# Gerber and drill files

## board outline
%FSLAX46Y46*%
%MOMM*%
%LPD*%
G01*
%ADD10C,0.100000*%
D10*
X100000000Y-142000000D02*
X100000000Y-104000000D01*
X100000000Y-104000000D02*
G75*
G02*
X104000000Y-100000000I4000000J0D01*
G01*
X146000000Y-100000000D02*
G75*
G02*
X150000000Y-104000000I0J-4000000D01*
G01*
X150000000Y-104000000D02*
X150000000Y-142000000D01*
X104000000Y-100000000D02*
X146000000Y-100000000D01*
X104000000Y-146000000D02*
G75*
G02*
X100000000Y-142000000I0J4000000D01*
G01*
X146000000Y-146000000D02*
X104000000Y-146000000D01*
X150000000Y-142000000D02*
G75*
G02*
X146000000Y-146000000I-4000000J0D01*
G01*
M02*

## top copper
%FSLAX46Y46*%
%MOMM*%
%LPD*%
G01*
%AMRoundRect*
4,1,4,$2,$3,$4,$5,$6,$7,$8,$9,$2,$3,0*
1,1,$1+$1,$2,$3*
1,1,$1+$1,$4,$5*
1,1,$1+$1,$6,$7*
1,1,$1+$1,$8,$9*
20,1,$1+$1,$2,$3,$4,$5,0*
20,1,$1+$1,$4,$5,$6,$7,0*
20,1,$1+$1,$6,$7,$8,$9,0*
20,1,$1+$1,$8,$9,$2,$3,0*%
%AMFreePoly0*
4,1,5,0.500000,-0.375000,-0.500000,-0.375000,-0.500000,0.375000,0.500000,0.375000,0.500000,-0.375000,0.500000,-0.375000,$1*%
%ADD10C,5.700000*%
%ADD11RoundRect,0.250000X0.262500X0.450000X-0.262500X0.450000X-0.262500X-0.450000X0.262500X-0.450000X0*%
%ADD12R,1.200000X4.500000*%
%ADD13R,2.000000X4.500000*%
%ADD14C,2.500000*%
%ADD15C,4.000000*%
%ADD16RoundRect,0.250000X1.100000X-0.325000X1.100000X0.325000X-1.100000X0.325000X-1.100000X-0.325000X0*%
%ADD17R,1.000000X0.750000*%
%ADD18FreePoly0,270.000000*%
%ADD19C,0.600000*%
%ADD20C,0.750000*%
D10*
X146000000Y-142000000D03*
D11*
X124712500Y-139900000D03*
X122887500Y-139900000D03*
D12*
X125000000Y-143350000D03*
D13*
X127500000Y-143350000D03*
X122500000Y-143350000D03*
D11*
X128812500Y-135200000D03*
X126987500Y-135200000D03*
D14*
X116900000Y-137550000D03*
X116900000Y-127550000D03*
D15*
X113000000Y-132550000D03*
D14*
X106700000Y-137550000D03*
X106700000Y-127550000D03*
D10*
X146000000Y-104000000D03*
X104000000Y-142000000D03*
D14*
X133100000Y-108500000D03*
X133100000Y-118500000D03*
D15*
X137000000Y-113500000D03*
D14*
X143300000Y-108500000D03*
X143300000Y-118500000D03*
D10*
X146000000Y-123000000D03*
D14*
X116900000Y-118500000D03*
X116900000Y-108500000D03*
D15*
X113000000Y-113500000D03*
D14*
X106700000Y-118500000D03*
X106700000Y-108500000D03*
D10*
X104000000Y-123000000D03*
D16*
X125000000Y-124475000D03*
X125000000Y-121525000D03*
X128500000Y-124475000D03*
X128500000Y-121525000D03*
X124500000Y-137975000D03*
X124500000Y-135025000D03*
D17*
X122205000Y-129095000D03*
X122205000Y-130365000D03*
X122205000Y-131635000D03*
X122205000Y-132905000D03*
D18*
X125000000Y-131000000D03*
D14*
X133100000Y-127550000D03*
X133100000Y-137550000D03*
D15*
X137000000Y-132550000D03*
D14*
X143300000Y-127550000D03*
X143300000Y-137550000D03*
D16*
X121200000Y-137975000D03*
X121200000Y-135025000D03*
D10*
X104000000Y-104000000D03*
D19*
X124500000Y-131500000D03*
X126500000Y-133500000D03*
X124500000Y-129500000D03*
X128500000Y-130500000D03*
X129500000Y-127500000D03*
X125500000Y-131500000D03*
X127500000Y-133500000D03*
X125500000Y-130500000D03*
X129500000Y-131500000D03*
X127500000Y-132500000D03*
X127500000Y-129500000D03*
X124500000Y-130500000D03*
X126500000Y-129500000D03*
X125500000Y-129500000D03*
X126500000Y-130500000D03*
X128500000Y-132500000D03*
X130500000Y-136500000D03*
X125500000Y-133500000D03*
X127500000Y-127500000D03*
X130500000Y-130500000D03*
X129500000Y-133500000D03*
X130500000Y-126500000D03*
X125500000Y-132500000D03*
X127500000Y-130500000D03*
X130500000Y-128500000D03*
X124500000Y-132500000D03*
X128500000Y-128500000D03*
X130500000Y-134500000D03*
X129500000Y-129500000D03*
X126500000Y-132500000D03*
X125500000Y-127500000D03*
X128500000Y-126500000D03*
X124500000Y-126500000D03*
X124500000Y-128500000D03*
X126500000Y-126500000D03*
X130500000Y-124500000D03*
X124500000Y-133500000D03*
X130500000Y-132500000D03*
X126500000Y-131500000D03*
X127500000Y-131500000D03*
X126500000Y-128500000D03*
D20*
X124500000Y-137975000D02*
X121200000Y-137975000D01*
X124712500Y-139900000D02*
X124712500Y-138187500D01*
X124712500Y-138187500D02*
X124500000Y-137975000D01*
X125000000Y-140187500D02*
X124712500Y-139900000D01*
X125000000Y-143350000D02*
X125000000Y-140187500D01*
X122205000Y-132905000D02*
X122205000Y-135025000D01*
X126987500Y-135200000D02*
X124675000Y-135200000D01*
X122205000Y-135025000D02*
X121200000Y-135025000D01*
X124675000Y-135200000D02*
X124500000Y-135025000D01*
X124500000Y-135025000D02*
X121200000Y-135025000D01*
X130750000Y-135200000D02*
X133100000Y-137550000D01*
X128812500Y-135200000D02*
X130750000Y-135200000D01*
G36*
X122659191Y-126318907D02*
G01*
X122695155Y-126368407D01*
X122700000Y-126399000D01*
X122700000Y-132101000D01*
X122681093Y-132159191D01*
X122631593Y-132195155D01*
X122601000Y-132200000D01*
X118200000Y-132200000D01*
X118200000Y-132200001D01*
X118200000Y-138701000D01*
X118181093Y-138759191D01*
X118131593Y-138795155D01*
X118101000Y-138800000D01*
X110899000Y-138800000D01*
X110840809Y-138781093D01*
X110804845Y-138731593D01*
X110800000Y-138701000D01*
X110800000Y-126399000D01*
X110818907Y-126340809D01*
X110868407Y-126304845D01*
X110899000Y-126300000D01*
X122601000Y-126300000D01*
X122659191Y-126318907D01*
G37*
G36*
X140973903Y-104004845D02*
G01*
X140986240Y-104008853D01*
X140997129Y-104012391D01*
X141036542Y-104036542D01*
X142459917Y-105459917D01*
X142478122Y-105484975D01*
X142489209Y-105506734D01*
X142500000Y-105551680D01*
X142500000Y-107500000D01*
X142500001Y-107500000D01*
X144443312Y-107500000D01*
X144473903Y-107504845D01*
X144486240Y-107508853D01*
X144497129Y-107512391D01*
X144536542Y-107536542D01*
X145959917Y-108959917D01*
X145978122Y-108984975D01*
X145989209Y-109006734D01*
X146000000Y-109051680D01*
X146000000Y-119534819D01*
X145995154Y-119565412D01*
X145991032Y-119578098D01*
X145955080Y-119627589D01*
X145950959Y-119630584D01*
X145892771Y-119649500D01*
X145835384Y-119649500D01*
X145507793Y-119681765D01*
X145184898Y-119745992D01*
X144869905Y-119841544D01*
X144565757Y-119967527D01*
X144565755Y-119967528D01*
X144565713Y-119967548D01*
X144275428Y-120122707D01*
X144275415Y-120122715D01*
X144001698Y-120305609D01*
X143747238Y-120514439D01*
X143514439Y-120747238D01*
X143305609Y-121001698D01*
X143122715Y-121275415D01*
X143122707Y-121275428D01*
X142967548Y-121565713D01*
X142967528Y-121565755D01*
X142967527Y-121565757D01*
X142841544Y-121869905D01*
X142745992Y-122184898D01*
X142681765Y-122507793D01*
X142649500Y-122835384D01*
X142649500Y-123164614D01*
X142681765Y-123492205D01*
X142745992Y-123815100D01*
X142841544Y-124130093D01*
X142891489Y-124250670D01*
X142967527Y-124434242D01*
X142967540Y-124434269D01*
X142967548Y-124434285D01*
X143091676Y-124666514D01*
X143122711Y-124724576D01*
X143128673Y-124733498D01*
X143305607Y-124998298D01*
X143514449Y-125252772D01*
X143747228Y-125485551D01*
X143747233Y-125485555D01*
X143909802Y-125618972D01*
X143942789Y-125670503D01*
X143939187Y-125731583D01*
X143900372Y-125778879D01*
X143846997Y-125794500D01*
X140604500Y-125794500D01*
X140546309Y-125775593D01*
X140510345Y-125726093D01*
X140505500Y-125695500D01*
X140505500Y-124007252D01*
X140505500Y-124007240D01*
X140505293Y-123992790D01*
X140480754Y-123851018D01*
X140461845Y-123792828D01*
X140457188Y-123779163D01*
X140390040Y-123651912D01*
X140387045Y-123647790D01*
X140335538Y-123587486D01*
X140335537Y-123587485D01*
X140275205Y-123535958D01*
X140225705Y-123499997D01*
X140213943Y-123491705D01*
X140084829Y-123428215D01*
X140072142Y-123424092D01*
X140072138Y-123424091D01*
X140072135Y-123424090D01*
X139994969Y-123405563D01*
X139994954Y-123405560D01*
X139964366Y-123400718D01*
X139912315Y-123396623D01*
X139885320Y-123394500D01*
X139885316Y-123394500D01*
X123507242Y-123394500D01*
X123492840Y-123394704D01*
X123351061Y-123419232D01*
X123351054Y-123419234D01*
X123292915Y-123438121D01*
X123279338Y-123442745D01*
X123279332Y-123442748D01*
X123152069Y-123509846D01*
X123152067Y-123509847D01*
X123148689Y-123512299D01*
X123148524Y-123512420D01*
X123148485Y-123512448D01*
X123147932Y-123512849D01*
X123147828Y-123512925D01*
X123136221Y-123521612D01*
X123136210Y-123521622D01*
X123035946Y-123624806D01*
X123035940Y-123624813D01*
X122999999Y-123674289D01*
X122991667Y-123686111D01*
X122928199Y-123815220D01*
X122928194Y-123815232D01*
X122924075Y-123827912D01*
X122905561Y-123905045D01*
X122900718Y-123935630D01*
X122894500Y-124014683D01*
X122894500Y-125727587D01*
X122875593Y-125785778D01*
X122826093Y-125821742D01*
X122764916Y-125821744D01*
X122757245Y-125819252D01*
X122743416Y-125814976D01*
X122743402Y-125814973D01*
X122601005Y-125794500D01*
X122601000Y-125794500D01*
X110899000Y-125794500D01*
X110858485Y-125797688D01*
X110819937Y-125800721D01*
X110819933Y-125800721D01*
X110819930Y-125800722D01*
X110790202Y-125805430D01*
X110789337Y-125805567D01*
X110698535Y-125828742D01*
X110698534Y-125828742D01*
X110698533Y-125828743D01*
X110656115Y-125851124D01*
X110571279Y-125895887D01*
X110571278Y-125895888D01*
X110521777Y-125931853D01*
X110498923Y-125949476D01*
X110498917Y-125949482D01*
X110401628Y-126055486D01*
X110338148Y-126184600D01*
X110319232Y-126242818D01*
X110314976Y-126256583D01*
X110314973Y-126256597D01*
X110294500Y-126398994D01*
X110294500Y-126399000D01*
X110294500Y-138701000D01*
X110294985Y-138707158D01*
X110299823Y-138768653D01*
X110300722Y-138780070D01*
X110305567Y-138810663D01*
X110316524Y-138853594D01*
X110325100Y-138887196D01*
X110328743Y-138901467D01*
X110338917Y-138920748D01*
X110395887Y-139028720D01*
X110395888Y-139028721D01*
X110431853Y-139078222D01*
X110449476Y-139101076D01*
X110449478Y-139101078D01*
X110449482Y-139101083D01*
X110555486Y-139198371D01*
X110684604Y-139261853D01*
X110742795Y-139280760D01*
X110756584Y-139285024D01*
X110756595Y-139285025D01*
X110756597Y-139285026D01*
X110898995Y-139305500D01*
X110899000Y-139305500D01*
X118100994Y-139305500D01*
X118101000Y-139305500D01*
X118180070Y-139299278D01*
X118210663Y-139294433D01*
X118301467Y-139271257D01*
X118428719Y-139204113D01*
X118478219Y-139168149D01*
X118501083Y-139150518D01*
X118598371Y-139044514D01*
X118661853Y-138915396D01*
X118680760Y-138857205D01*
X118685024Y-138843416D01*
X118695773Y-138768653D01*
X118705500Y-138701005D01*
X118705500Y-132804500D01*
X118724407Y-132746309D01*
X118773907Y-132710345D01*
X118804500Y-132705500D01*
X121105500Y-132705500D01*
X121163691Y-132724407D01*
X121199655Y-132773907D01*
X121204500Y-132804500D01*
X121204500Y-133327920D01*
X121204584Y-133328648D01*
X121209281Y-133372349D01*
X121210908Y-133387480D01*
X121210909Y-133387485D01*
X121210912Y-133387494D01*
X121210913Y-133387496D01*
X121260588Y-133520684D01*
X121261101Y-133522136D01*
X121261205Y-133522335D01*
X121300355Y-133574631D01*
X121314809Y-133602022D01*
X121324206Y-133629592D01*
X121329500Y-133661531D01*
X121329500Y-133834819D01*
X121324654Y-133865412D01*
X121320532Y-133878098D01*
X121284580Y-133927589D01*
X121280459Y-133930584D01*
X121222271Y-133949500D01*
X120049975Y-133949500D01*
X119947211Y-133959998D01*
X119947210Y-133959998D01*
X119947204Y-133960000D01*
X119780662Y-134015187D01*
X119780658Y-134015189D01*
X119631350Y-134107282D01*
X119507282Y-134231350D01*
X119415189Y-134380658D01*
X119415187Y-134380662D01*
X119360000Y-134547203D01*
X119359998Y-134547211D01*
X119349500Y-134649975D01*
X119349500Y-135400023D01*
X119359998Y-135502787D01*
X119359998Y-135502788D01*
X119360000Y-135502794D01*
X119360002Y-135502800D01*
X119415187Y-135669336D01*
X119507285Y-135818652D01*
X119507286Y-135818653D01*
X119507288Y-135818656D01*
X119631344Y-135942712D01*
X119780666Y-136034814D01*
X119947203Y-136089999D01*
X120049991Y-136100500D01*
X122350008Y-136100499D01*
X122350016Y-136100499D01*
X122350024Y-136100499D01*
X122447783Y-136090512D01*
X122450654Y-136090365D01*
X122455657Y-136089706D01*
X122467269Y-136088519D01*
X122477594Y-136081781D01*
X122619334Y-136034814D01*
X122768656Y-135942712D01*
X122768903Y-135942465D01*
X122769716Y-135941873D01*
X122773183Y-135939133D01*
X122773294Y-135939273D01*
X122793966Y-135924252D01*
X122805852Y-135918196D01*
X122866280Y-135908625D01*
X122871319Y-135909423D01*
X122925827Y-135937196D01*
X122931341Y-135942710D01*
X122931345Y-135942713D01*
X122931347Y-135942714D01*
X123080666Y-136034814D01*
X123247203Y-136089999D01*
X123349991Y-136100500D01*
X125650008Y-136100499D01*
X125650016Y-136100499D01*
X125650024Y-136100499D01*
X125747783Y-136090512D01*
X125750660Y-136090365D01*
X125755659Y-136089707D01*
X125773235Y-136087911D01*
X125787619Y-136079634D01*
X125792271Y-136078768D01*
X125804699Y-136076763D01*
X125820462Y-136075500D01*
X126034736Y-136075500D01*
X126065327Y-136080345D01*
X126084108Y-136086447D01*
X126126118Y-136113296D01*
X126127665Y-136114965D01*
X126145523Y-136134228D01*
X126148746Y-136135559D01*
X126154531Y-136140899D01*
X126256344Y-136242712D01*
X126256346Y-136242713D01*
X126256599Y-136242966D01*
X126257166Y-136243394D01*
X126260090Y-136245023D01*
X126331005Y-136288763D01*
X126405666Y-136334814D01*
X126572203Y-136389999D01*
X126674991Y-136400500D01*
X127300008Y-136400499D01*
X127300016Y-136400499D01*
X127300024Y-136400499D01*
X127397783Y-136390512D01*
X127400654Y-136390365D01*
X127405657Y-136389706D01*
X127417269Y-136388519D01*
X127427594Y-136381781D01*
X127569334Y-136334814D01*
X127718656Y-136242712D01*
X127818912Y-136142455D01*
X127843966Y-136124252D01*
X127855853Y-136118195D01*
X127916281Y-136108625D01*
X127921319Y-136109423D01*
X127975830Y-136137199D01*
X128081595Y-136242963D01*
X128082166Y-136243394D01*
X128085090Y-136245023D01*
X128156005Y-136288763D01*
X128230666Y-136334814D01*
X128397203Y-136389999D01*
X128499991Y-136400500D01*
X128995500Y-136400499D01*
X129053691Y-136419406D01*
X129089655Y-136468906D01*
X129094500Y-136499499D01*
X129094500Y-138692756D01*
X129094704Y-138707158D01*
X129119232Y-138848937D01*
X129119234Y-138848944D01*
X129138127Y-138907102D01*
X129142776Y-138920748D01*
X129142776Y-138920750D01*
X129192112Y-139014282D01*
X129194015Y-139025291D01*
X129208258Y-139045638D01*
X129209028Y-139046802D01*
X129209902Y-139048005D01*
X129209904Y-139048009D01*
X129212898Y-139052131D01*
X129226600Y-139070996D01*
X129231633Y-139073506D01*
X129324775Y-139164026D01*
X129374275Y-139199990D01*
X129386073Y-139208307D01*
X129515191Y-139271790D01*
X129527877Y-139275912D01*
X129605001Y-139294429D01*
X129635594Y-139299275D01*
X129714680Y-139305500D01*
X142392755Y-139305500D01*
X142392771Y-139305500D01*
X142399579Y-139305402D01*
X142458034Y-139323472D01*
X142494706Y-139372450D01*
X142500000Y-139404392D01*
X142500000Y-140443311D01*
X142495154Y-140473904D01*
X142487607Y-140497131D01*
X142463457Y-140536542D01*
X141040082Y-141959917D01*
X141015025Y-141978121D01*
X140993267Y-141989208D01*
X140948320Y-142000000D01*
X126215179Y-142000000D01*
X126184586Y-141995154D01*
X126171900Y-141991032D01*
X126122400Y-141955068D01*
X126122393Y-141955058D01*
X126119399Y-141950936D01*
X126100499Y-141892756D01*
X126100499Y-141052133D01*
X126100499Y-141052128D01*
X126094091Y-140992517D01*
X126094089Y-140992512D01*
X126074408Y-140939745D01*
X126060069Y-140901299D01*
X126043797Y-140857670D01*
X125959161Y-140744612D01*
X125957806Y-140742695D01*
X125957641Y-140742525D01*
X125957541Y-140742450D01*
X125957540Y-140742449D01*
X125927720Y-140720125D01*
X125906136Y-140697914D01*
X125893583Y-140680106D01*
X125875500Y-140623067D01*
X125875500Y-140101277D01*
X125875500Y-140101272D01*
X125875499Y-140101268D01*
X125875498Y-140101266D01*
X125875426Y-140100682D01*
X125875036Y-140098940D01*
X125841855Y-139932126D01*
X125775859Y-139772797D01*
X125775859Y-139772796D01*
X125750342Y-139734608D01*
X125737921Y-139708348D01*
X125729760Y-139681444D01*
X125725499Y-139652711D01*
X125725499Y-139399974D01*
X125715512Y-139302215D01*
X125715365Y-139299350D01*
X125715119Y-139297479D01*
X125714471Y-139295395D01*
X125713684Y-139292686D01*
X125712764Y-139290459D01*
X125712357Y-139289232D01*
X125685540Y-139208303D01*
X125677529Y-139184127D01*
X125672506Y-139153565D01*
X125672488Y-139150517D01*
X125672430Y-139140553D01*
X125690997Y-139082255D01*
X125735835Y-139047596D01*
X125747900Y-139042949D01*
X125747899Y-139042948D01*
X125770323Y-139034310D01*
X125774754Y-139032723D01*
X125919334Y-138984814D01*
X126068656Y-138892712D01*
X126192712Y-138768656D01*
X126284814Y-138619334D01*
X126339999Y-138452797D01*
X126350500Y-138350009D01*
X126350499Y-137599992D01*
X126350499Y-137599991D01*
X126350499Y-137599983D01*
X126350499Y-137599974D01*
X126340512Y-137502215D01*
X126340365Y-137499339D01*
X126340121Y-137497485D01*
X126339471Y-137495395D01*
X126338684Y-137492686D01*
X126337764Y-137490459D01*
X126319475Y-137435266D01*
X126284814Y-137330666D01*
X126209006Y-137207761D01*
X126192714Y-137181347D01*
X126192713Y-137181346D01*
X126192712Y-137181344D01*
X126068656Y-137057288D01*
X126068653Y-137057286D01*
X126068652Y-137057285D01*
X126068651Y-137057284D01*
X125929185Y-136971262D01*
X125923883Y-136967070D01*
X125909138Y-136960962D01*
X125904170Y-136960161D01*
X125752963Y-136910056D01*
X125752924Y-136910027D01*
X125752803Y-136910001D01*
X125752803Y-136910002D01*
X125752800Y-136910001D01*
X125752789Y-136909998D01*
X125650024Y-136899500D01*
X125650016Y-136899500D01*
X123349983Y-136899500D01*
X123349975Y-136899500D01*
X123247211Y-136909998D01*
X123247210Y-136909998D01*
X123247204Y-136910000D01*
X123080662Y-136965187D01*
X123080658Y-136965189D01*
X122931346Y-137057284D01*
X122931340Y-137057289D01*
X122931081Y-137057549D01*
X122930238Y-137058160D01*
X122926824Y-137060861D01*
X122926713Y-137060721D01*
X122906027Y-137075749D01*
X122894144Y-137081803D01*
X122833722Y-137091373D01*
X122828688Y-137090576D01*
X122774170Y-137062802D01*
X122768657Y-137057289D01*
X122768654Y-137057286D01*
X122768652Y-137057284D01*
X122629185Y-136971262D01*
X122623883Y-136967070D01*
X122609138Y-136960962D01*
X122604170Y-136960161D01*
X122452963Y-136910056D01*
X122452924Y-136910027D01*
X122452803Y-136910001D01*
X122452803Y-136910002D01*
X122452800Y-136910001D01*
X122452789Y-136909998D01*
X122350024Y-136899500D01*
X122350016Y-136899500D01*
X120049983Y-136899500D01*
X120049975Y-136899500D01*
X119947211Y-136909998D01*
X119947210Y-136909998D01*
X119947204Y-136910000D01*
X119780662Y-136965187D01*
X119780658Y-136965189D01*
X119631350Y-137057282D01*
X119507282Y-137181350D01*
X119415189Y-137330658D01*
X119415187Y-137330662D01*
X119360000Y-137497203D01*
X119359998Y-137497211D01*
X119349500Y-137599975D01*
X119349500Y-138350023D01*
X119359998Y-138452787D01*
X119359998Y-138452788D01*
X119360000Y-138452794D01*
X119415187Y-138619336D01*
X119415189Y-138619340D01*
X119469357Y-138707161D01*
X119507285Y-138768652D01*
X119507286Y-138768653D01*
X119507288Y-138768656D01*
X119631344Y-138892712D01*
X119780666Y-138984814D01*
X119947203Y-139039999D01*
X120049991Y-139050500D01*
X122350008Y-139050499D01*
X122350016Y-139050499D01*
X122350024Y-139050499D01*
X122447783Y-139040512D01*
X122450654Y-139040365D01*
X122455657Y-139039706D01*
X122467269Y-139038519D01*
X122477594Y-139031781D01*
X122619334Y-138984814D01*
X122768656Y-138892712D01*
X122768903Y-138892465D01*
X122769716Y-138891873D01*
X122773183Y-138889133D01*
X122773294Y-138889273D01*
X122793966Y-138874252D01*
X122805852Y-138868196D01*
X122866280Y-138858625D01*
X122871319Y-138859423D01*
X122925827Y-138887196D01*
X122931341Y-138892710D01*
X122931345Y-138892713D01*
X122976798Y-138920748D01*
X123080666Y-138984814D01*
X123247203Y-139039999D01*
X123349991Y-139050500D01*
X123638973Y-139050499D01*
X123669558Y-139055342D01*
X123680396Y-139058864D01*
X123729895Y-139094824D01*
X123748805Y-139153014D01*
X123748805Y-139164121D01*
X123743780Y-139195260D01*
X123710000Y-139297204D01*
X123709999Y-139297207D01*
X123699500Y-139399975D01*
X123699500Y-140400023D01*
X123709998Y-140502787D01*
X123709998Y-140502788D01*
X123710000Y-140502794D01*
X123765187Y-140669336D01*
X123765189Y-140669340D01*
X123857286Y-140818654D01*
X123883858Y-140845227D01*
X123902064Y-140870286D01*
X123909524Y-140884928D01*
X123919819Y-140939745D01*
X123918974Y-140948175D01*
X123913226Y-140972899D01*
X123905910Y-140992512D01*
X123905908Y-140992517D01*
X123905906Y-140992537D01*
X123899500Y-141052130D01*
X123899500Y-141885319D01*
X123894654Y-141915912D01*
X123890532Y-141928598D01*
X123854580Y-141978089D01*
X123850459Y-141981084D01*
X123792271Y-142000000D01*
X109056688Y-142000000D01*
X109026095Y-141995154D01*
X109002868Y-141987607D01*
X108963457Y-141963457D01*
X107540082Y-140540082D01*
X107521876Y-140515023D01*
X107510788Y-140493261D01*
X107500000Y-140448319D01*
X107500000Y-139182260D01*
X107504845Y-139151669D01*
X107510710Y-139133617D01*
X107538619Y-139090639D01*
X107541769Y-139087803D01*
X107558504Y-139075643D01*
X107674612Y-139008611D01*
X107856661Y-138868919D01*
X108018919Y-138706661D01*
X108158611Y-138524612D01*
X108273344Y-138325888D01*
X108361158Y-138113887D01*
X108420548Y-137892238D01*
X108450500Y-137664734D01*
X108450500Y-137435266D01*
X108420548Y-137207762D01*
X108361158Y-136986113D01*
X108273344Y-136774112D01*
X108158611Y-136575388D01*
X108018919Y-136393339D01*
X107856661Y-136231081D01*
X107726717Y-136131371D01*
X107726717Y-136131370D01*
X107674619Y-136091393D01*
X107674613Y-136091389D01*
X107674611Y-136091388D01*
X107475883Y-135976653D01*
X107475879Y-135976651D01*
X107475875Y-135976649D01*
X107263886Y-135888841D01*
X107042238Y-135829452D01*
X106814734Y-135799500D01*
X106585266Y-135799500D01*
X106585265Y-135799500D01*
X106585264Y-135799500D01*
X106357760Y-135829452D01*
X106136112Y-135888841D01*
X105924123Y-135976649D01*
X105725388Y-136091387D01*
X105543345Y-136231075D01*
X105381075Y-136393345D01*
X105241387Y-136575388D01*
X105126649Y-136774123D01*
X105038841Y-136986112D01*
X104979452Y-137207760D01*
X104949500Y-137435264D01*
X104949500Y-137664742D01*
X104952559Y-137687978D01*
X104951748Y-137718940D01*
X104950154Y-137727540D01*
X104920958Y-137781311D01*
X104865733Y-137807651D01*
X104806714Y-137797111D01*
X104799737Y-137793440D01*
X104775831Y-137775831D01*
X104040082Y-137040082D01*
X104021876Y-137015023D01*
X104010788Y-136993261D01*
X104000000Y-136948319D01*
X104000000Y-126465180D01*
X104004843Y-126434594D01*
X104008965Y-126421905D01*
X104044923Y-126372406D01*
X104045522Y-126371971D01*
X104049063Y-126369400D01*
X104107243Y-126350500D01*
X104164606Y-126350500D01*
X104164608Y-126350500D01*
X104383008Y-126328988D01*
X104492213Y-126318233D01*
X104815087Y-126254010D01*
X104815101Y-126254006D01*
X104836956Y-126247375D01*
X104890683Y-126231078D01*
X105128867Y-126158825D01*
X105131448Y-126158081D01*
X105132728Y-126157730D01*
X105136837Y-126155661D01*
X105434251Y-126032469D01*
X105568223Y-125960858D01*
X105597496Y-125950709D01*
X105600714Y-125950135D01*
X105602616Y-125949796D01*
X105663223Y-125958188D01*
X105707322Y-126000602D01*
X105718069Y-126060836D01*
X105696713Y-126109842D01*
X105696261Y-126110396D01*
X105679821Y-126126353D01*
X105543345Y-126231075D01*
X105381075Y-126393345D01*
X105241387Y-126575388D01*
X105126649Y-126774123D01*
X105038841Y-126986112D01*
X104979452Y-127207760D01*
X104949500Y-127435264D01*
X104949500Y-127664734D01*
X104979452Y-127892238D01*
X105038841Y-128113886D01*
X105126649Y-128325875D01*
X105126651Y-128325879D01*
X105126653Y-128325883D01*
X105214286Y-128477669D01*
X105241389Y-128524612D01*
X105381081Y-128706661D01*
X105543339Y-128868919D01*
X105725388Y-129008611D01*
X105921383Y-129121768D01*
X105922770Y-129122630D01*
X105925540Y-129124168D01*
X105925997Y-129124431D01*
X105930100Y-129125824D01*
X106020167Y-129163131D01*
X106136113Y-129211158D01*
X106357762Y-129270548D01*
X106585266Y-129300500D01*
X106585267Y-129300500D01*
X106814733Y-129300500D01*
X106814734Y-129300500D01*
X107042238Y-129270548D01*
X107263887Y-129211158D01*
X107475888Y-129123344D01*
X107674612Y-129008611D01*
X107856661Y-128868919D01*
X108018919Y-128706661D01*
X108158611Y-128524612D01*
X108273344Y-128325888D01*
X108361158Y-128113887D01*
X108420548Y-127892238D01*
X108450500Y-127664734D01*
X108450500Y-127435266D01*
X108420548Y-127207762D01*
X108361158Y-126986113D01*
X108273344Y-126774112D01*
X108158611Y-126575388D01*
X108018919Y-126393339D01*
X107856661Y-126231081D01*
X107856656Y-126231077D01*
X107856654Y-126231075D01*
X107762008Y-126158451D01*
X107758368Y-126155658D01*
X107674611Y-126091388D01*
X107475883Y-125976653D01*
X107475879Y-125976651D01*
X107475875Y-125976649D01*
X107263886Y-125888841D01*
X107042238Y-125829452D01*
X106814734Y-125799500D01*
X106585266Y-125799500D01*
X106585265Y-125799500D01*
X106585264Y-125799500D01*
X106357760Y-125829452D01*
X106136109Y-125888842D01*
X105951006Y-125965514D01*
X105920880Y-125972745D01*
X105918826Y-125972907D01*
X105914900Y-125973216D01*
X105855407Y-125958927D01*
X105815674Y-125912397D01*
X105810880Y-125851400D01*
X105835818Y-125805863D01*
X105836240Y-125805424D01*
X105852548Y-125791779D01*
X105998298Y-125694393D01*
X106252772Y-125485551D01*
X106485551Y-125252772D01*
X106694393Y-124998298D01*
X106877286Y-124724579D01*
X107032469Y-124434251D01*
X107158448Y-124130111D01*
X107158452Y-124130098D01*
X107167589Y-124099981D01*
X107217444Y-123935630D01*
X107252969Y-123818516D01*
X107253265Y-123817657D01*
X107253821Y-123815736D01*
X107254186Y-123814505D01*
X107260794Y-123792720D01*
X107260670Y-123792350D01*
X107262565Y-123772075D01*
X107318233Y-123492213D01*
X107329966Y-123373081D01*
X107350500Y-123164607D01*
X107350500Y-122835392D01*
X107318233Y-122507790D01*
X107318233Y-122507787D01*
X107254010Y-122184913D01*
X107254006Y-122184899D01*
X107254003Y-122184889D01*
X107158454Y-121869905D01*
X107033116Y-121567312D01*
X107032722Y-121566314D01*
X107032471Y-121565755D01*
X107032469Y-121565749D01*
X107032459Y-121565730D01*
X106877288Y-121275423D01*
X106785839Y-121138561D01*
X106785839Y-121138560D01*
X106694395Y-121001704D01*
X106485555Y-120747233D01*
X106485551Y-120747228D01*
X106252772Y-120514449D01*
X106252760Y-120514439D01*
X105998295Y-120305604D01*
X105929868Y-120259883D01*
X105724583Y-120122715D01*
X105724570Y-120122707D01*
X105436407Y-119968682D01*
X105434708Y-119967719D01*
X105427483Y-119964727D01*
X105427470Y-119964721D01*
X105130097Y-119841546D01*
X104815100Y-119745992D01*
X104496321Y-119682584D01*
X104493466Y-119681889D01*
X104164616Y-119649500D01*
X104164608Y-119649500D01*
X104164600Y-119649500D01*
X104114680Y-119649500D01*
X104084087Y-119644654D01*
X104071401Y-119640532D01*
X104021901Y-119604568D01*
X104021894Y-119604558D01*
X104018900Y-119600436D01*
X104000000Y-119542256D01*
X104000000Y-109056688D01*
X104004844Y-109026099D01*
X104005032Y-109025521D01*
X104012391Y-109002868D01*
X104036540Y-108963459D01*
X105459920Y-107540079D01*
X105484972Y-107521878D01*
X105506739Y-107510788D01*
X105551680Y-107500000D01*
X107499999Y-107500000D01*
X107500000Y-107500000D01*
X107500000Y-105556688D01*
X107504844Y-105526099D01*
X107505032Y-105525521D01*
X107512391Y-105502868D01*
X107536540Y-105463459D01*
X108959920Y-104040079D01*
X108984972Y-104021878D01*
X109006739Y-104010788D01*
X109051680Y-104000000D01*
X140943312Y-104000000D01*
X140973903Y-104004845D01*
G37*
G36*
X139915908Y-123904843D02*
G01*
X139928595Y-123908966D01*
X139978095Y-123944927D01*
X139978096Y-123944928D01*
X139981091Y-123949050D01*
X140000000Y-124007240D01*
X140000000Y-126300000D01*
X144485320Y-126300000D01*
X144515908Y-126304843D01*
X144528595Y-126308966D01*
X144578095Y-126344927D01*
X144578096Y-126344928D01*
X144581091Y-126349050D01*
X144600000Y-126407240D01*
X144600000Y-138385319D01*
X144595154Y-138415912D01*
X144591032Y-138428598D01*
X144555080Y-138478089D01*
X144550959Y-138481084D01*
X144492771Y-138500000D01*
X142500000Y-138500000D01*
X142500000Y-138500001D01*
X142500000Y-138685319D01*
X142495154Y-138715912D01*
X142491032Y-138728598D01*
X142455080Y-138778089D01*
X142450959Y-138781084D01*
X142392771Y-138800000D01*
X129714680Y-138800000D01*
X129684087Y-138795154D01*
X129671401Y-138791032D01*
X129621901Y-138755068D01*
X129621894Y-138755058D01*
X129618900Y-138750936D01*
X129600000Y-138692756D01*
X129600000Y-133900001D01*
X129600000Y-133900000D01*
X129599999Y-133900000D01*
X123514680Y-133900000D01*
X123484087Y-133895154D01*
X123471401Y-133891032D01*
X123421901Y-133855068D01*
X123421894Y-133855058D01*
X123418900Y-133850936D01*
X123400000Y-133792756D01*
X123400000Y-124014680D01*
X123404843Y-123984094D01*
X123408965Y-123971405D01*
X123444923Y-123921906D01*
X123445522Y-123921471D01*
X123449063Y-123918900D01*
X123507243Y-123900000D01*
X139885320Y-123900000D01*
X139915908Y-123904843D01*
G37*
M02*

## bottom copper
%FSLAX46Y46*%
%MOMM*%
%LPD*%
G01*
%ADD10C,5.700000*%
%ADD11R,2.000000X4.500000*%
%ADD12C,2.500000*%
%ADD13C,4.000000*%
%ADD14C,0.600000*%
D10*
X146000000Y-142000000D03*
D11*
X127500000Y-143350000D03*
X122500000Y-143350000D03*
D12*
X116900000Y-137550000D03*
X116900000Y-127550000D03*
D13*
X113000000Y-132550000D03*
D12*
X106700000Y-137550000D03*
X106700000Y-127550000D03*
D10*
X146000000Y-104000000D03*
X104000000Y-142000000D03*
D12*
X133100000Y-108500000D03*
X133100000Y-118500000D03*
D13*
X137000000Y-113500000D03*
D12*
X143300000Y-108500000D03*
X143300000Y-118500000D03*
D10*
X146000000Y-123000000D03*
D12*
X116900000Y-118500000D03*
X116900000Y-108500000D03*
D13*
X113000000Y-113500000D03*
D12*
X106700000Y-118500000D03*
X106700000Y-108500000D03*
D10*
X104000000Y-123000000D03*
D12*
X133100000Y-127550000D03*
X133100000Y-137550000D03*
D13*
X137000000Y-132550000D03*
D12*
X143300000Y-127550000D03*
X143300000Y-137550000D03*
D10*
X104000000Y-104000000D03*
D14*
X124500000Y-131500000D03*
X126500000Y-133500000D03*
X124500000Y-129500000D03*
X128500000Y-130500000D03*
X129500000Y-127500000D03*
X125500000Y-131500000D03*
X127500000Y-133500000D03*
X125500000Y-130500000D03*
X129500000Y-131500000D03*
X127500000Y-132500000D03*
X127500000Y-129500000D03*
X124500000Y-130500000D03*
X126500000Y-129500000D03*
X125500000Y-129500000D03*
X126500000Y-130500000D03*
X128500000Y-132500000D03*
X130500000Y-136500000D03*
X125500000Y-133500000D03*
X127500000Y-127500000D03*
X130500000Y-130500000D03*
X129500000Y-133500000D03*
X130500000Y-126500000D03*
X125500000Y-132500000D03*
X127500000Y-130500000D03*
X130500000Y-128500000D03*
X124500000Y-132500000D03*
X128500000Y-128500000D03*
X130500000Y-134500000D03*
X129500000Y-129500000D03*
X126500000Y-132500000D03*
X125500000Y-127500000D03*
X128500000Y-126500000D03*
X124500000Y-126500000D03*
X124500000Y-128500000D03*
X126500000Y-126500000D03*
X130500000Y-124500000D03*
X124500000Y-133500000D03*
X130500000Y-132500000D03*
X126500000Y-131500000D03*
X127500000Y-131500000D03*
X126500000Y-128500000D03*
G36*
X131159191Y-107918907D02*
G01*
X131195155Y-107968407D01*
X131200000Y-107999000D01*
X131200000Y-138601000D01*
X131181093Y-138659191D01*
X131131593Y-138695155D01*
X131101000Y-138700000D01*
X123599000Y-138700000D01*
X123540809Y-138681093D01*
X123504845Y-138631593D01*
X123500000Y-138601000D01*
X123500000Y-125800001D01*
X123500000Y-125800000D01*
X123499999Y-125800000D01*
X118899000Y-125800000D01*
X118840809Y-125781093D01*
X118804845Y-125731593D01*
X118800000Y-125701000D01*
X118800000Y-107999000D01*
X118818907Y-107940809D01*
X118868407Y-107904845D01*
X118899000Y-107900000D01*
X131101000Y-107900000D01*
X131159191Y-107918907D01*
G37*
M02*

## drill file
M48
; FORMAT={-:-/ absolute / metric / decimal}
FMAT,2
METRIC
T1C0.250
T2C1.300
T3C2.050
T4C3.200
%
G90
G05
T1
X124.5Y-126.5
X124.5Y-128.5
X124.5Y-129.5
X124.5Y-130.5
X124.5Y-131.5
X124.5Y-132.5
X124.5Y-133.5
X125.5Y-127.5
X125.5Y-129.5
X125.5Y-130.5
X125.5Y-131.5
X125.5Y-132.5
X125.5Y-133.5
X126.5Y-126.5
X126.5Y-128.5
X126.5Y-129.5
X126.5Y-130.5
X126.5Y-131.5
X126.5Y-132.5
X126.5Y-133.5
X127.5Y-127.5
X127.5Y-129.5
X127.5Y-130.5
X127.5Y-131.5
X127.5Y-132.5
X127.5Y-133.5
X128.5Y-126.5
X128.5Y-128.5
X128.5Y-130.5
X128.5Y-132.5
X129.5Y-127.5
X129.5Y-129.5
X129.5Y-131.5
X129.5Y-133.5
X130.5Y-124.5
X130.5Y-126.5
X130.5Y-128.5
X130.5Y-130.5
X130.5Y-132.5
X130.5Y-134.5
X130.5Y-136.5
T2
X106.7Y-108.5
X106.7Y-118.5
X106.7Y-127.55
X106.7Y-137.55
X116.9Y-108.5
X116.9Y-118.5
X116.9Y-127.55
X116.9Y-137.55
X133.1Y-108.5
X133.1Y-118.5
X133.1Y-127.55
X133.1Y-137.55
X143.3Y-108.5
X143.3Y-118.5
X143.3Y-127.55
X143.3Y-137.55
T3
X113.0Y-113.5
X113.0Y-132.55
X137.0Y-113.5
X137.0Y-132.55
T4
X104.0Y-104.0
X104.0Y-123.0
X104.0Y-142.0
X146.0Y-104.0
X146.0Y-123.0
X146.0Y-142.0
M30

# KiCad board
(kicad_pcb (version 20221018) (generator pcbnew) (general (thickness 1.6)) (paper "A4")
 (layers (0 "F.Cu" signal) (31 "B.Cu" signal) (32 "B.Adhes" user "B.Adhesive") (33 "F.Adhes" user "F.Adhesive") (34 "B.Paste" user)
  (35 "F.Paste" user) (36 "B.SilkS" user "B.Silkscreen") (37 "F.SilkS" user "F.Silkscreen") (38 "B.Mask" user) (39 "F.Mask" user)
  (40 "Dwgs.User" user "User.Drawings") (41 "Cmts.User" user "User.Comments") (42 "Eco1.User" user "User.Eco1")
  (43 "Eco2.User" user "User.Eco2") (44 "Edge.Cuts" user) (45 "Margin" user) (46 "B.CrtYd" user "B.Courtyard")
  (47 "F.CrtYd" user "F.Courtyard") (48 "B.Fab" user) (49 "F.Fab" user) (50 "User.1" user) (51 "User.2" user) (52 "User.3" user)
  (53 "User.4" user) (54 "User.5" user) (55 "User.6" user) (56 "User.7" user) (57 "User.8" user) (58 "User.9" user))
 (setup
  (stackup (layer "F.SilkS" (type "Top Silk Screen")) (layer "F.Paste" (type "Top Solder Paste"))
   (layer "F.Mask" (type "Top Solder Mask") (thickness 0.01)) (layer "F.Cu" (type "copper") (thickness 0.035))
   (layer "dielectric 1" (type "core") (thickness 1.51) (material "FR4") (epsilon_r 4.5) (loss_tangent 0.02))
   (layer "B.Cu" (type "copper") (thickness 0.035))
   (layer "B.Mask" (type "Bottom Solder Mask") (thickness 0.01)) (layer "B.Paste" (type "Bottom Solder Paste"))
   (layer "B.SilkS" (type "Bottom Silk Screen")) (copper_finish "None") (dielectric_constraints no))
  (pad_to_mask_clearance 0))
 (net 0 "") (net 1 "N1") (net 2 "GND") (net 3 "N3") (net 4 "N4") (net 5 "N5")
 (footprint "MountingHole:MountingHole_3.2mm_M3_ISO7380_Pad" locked (layer "F.Cu") (at 146 142)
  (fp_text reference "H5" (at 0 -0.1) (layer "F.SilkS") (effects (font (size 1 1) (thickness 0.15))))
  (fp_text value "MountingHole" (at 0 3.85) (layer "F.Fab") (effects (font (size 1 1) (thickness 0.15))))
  (pad "1" thru_hole circle locked (at 0 0) (size 5.7 5.7) (drill 3.2) (layers "*.Cu" "*.Mask")))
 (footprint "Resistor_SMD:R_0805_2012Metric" (layer "F.Cu") (at 123.8 139.9 180)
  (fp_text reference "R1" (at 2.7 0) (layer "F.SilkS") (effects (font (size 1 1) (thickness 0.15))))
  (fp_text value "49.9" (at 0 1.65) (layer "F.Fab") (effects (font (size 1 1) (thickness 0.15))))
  (pad "1" smd roundrect (at -0.9125 0 180) (size 1.025 1.4) (layers "F.Cu" "F.Paste" "F.Mask") (roundrect_rratio 0.243902439) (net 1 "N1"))
  (pad "2" smd roundrect (at 0.9125 0 180) (size 1.025 1.4) (layers "F.Cu" "F.Paste" "F.Mask") (roundrect_rratio 0.243902439) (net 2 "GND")))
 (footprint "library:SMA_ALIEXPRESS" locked (layer "F.Cu") (at 125 145.6 180)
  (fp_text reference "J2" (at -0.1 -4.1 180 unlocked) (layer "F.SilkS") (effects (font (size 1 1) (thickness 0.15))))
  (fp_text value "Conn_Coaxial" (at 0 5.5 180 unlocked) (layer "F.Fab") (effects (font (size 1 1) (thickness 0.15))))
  (pad "1" smd rect locked (at 0 2.25 180) (size 1.2 4.5) (layers "F.Cu" "F.Paste" "F.Mask") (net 1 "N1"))
  (pad "2" smd rect locked (at -2.5 2.25 180) (size 2 4.5) (layers "F.Cu" "F.Paste" "F.Mask") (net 2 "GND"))
  (pad "2" smd rect locked (at -2.5 2.25 180) (size 2 4.5) (layers "B.Cu" "B.Paste" "B.Mask") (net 2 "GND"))
  (pad "2" smd rect locked (at 2.5 2.25 180) (size 2 4.5) (layers "F.Cu" "F.Paste" "F.Mask") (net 2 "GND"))
  (pad "2" smd rect locked (at 2.5 2.25 180) (size 2 4.5) (layers "B.Cu" "B.Paste" "B.Mask") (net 2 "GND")))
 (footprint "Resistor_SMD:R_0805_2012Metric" (layer "F.Cu") (at 127.9 135.2 180)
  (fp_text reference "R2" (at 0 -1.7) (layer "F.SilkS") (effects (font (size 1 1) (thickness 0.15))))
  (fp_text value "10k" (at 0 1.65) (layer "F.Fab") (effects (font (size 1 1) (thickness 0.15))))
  (pad "1" smd roundrect (at -0.9125 0 180) (size 1.025 1.4) (layers "F.Cu" "F.Paste" "F.Mask") (roundrect_rratio 0.243902439) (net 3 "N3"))
  (pad "2" smd roundrect (at 0.9125 0 180) (size 1.025 1.4) (layers "F.Cu" "F.Paste" "F.Mask") (roundrect_rratio 0.243902439) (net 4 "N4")))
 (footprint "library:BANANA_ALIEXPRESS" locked (layer "F.Cu") (at 113 132.55 180)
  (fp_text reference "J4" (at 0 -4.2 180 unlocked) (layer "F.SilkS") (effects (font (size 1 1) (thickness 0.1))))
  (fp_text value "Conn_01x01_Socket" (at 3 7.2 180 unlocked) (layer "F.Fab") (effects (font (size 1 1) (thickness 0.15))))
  (pad "1" thru_hole circle locked (at -3.9 -5 180) (size 2.5 2.5) (drill 1.3) (layers "*.Cu" "*.Mask") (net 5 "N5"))
  (pad "1" thru_hole circle locked (at -3.9 5 180) (size 2.5 2.5) (drill 1.3) (layers "*.Cu" "*.Mask") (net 5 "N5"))
  (pad "1" thru_hole circle locked (at 0 0 180) (size 4 4) (drill 2.05) (layers "*.Cu" "*.Mask") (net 5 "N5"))
  (pad "1" thru_hole circle locked (at 6.3 -5 180) (size 2.5 2.5) (drill 1.3) (layers "*.Cu" "*.Mask") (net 5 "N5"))
  (pad "1" thru_hole circle locked (at 6.3 5 180) (size 2.5 2.5) (drill 1.3) (layers "*.Cu" "*.Mask") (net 5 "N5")))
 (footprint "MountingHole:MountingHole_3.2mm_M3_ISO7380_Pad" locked (layer "F.Cu") (at 146 104)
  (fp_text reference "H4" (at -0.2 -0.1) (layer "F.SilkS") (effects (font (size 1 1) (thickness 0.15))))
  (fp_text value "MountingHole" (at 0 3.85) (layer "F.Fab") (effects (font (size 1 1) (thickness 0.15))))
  (pad "1" thru_hole circle locked (at 0 0) (size 5.7 5.7) (drill 3.2) (layers "*.Cu" "*.Mask")))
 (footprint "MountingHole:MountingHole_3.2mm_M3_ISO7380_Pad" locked (layer "F.Cu") (at 104 142)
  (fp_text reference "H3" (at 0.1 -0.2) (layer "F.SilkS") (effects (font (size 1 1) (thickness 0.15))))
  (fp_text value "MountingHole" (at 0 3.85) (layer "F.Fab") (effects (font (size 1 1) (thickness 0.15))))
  (pad "1" thru_hole circle locked (at 0 0) (size 5.7 5.7) (drill 3.2) (layers "*.Cu" "*.Mask")))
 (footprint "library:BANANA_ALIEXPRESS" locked (layer "F.Cu") (at 137 113.5)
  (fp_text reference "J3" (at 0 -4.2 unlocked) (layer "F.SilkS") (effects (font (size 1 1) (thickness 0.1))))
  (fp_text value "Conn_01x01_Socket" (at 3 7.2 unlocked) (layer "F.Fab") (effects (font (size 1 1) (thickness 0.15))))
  (pad "1" thru_hole circle locked (at -3.9 -5) (size 2.5 2.5) (drill 1.3) (layers "*.Cu" "*.Mask") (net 2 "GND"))
  (pad "1" thru_hole circle locked (at -3.9 5) (size 2.5 2.5) (drill 1.3) (layers "*.Cu" "*.Mask") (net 2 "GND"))
  (pad "1" thru_hole circle locked (at 0 0) (size 4 4) (drill 2.05) (layers "*.Cu" "*.Mask") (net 2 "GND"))
  (pad "1" thru_hole circle locked (at 6.3 -5) (size 2.5 2.5) (drill 1.3) (layers "*.Cu" "*.Mask") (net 2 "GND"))
  (pad "1" thru_hole circle locked (at 6.3 5) (size 2.5 2.5) (drill 1.3) (layers "*.Cu" "*.Mask") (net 2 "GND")))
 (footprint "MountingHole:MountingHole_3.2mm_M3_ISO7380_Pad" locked (layer "F.Cu") (at 146 123)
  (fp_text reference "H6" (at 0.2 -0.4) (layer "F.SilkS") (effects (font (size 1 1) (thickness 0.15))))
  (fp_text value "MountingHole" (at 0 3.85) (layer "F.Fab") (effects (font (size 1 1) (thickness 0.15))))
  (pad "1" thru_hole circle locked (at 0 0) (size 5.7 5.7) (drill 3.2) (layers "*.Cu" "*.Mask")))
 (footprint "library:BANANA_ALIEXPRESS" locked (layer "F.Cu") (at 113 113.5 180)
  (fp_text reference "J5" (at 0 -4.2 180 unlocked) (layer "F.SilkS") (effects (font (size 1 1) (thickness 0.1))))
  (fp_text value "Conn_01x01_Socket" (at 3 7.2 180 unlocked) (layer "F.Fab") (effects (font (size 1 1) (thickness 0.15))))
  (pad "1" thru_hole circle locked (at -3.9 -5 180) (size 2.5 2.5) (drill 1.3) (layers "*.Cu" "*.Mask") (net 2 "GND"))
  (pad "1" thru_hole circle locked (at -3.9 5 180) (size 2.5 2.5) (drill 1.3) (layers "*.Cu" "*.Mask") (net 2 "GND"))
  (pad "1" thru_hole circle locked (at 0 0 180) (size 4 4) (drill 2.05) (layers "*.Cu" "*.Mask") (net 2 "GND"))
  (pad "1" thru_hole circle locked (at 6.3 -5 180) (size 2.5 2.5) (drill 1.3) (layers "*.Cu" "*.Mask") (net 2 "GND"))
  (pad "1" thru_hole circle locked (at 6.3 5 180) (size 2.5 2.5) (drill 1.3) (layers "*.Cu" "*.Mask") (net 2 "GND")))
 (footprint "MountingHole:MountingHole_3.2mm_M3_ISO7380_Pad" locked (layer "F.Cu") (at 104 123)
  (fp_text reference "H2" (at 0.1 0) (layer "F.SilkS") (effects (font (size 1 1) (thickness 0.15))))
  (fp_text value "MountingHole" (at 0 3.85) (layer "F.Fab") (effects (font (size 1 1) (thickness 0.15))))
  (pad "1" thru_hole circle locked (at 0 0) (size 5.7 5.7) (drill 3.2) (layers "*.Cu" "*.Mask")))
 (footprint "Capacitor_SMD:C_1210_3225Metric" (layer "F.Cu") (at 125 123 90)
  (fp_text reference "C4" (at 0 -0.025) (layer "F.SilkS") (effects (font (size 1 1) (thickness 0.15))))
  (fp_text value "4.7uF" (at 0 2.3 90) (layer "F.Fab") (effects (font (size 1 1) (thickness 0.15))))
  (pad "1" smd roundrect (at -1.475 0 90) (size 1.15 2.7) (layers "F.Cu" "F.Paste" "F.Mask") (roundrect_rratio 0.2173913043) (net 3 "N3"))
  (pad "2" smd roundrect (at 1.475 0 90) (size 1.15 2.7) (layers "F.Cu" "F.Paste" "F.Mask") (roundrect_rratio 0.2173913043) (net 2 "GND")))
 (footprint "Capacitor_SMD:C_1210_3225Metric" (layer "F.Cu") (at 128.5 123 90)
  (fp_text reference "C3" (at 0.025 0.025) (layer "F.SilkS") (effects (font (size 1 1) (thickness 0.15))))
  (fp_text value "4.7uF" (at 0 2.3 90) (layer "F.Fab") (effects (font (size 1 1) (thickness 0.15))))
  (pad "1" smd roundrect (at -1.475 0 90) (size 1.15 2.7) (layers "F.Cu" "F.Paste" "F.Mask") (roundrect_rratio 0.2173913043) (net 3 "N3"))
  (pad "2" smd roundrect (at 1.475 0 90) (size 1.15 2.7) (layers "F.Cu" "F.Paste" "F.Mask") (roundrect_rratio 0.2173913043) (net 2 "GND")))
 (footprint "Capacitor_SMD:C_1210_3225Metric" (layer "F.Cu") (at 124.5 136.5 90)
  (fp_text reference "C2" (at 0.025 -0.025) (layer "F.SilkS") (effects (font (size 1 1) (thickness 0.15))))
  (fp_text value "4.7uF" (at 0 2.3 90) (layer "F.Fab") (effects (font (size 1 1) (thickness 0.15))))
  (pad "1" smd roundrect (at -1.475 0 90) (size 1.15 2.7) (layers "F.Cu" "F.Paste" "F.Mask") (roundrect_rratio 0.2173913043) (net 1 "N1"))
  (pad "2" smd roundrect (at 1.475 0 90) (size 1.15 2.7) (layers "F.Cu" "F.Paste" "F.Mask") (roundrect_rratio 0.2173913043) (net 4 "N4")))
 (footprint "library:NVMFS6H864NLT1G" (layer "F.Cu") (at 125 131)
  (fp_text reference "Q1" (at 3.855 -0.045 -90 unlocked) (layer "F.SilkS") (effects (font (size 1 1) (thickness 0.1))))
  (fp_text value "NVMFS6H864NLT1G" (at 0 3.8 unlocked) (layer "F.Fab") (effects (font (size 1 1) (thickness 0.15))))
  (pad "1" smd rect (at -2.795 -1.905) (size 1 0.75) (layers "F.Cu" "F.Paste" "F.Mask") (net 5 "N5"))
  (pad "2" smd rect (at -2.795 -0.635) (size 1 0.75) (layers "F.Cu" "F.Paste" "F.Mask") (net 5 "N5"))
  (pad "3" smd rect (at -2.795 0.635) (size 1 0.75) (layers "F.Cu" "F.Paste" "F.Mask") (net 5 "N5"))
  (pad "4" smd rect (at -2.795 1.905) (size 1 0.75) (layers "F.Cu" "F.Paste" "F.Mask") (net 4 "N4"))
  (pad "5" smd custom (at 0 0 270) (size 1 0.75) (layers "F.Cu" "F.Paste" "F.Mask") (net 3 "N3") (options (clearance outline) (anchor rect))
   (primitives)))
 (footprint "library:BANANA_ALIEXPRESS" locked (layer "F.Cu") (at 137 132.55)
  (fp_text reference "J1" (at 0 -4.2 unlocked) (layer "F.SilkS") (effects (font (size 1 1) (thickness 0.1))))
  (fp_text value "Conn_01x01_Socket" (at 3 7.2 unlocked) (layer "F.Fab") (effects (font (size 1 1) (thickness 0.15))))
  (pad "1" thru_hole circle locked (at -3.9 -5) (size 2.5 2.5) (drill 1.3) (layers "*.Cu" "*.Mask") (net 3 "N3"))
  (pad "1" thru_hole circle locked (at -3.9 5) (size 2.5 2.5) (drill 1.3) (layers "*.Cu" "*.Mask") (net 3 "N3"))
  (pad "1" thru_hole circle locked (at 0 0) (size 4 4) (drill 2.05) (layers "*.Cu" "*.Mask") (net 3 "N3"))
  (pad "1" thru_hole circle locked (at 6.3 -5) (size 2.5 2.5) (drill 1.3) (layers "*.Cu" "*.Mask") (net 3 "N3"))
  (pad "1" thru_hole circle locked (at 6.3 5) (size 2.5 2.5) (drill 1.3) (layers "*.Cu" "*.Mask") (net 3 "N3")))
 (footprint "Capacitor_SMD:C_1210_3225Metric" (layer "F.Cu") (at 121.2 136.5 90)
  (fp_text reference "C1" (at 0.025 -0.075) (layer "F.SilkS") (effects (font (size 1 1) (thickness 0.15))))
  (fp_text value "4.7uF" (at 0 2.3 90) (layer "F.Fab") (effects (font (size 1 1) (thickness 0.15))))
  (pad "1" smd roundrect (at -1.475 0 90) (size 1.15 2.7) (layers "F.Cu" "F.Paste" "F.Mask") (roundrect_rratio 0.2173913043) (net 1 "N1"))
  (pad "2" smd roundrect (at 1.475 0 90) (size 1.15 2.7) (layers "F.Cu" "F.Paste" "F.Mask") (roundrect_rratio 0.2173913043) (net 4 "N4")))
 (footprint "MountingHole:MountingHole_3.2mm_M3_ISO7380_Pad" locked (layer "F.Cu") (at 104 104)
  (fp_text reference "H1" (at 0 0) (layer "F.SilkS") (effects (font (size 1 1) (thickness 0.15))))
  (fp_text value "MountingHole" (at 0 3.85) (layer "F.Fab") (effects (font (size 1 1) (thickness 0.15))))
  (pad "1" thru_hole circle locked (at 0 0) (size 5.7 5.7) (drill 3.2) (layers "*.Cu" "*.Mask")))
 (gr_line (start 100 142) (end 100 104) (stroke (width 0.1) (type default)) (layer "Edge.Cuts"))
 (gr_arc (start 100 104) (mid 101.171573 101.171573) (end 104 100) (stroke (width 0.1) (type default)) (layer "Edge.Cuts"))
 (gr_arc (start 146 100) (mid 148.828427 101.171573) (end 150 104) (stroke (width 0.1) (type default)) (layer "Edge.Cuts"))
 (gr_line (start 150 104) (end 150 142) (stroke (width 0.1) (type default)) (layer "Edge.Cuts"))
 (gr_line (start 104 100) (end 146 100) (stroke (width 0.1) (type default)) (layer "Edge.Cuts"))
 (gr_arc (start 104 146) (mid 101.171573 144.828427) (end 100 142) (stroke (width 0.1) (type default)) (layer "Edge.Cuts"))
 (gr_line (start 146 146) (end 104 146) (stroke (width 0.1) (type default)) (layer "Edge.Cuts"))
 (gr_arc (start 150 142) (mid 148.828427 144.828427) (end 146 146) (stroke (width 0.1) (type default)) (layer "Edge.Cuts"))
 (segment (start 124.5 137.975) (end 121.2 137.975) (width 0.75) (layer "F.Cu") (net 1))
 (segment (start 124.7125 139.9) (end 124.7125 138.1875) (width 0.75) (layer "F.Cu") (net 1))
 (segment (start 124.7125 138.1875) (end 124.5 137.975) (width 0.75) (layer "F.Cu") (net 1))
 (segment (start 125 140.1875) (end 124.7125 139.9) (width 0.75) (layer "F.Cu") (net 1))
 (segment (start 125 143.35) (end 125 140.1875) (width 0.75) (layer "F.Cu") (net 1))
 (segment (start 122.205 132.905) (end 122.205 135.025) (width 0.75) (layer "F.Cu") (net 4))
 (segment (start 126.9875 135.2) (end 124.675 135.2) (width 0.75) (layer "F.Cu") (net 4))
 (segment (start 122.205 135.025) (end 121.2 135.025) (width 0.75) (layer "F.Cu") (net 4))
 (segment (start 124.675 135.2) (end 124.5 135.025) (width 0.75) (layer "F.Cu") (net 4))
 (segment (start 124.5 135.025) (end 121.2 135.025) (width 0.75) (layer "F.Cu") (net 4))
 (segment (start 130.75 135.2) (end 133.1 137.55) (width 0.75) (layer "F.Cu") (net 3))
 (segment (start 128.8125 135.2) (end 130.75 135.2) (width 0.75) (layer "F.Cu") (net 3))
 (via (at 124.5 131.5) (size 0.6) (drill 0.25) (layers "F.Cu" "B.Cu") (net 3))
 (via (at 126.5 133.5) (size 0.6) (drill 0.25) (layers "F.Cu" "B.Cu") (free) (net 3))
 (via (at 124.5 129.5) (size 0.6) (drill 0.25) (layers "F.Cu" "B.Cu") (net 3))
 (via (at 128.5 130.5) (size 0.6) (drill 0.25) (layers "F.Cu" "B.Cu") (free) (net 3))
 (via (at 129.5 127.5) (size 0.6) (drill 0.25) (layers "F.Cu" "B.Cu") (free) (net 3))
 (via (at 125.5 131.5) (size 0.6) (drill 0.25) (layers "F.Cu" "B.Cu") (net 3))
 (via (at 127.5 133.5) (size 0.6) (drill 0.25) (layers "F.Cu" "B.Cu") (free) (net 3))
 (via (at 125.5 130.5) (size 0.6) (drill 0.25) (layers "F.Cu" "B.Cu") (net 3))
 (via (at 129.5 131.5) (size 0.6) (drill 0.25) (layers "F.Cu" "B.Cu") (free) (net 3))
 (via (at 127.5 132.5) (size 0.6) (drill 0.25) (layers "F.Cu" "B.Cu") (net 3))
 (via (at 127.5 129.5) (size 0.6) (drill 0.25) (layers "F.Cu" "B.Cu") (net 3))
 (via (at 124.5 130.5) (size 0.6) (drill 0.25) (layers "F.Cu" "B.Cu") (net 3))
 (via (at 126.5 129.5) (size 0.6) (drill 0.25) (layers "F.Cu" "B.Cu") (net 3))
 (via (at 125.5 129.5) (size 0.6) (drill 0.25) (layers "F.Cu" "B.Cu") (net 3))
 (via (at 126.5 130.5) (size 0.6) (drill 0.25) (layers "F.Cu" "B.Cu") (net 3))
 (via (at 128.5 132.5) (size 0.6) (drill 0.25) (layers "F.Cu" "B.Cu") (free) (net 3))
 (via (at 130.5 136.5) (size 0.6) (drill 0.25) (layers "F.Cu" "B.Cu") (free) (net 3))
 (via (at 125.5 133.5) (size 0.6) (drill 0.25) (layers "F.Cu" "B.Cu") (free) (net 3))
 (via (at 127.5 127.5) (size 0.6) (drill 0.25) (layers "F.Cu" "B.Cu") (free) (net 3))
 (via (at 130.5 130.5) (size 0.6) (drill 0.25) (layers "F.Cu" "B.Cu") (free) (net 3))
 (via (at 129.5 133.5) (size 0.6) (drill 0.25) (layers "F.Cu" "B.Cu") (free) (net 3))
 (via (at 130.5 126.5) (size 0.6) (drill 0.25) (layers "F.Cu" "B.Cu") (free) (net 3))
 (via (at 125.5 132.5) (size 0.6) (drill 0.25) (layers "F.Cu" "B.Cu") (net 3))
 (via (at 127.5 130.5) (size 0.6) (drill 0.25) (layers "F.Cu" "B.Cu") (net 3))
 (via (at 130.5 128.5) (size 0.6) (drill 0.25) (layers "F.Cu" "B.Cu") (free) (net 3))
 (via (at 124.5 132.5) (size 0.6) (drill 0.25) (layers "F.Cu" "B.Cu") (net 3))
 (via (at 128.5 128.5) (size 0.6) (drill 0.25) (layers "F.Cu" "B.Cu") (free) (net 3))
 (via (at 130.5 134.5) (size 0.6) (drill 0.25) (layers "F.Cu" "B.Cu") (free) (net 3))
 (via (at 129.5 129.5) (size 0.6) (drill 0.25) (layers "F.Cu" "B.Cu") (free) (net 3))
 (via (at 126.5 132.5) (size 0.6) (drill 0.25) (layers "F.Cu" "B.Cu") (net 3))
 (via (at 125.5 127.5) (size 0.6) (drill 0.25) (layers "F.Cu" "B.Cu") (free) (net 3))
 (via (at 128.5 126.5) (size 0.6) (drill 0.25) (layers "F.Cu" "B.Cu") (free) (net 3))
 (via (at 124.5 126.5) (size 0.6) (drill 0.25) (layers "F.Cu" "B.Cu") (free) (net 3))
 (via (at 124.5 128.5) (size 0.6) (drill 0.25) (layers "F.Cu" "B.Cu") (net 3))
 (via (at 126.5 126.5) (size 0.6) (drill 0.25) (layers "F.Cu" "B.Cu") (free) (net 3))
 (via (at 130.5 124.5) (size 0.6) (drill 0.25) (layers "F.Cu" "B.Cu") (free) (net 3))
 (via (at 124.5 133.5) (size 0.6) (drill 0.25) (layers "F.Cu" "B.Cu") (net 3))
 (via (at 130.5 132.5) (size 0.6) (drill 0.25) (layers "F.Cu" "B.Cu") (free) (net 3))
 (via (at 126.5 131.5) (size 0.6) (drill 0.25) (layers "F.Cu" "B.Cu") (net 3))
 (via (at 127.5 131.5) (size 0.6) (drill 0.25) (layers "F.Cu" "B.Cu") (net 3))
 (via (at 126.5 128.5) (size 0.6) (drill 0.25) (layers "F.Cu" "B.Cu") (free) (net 3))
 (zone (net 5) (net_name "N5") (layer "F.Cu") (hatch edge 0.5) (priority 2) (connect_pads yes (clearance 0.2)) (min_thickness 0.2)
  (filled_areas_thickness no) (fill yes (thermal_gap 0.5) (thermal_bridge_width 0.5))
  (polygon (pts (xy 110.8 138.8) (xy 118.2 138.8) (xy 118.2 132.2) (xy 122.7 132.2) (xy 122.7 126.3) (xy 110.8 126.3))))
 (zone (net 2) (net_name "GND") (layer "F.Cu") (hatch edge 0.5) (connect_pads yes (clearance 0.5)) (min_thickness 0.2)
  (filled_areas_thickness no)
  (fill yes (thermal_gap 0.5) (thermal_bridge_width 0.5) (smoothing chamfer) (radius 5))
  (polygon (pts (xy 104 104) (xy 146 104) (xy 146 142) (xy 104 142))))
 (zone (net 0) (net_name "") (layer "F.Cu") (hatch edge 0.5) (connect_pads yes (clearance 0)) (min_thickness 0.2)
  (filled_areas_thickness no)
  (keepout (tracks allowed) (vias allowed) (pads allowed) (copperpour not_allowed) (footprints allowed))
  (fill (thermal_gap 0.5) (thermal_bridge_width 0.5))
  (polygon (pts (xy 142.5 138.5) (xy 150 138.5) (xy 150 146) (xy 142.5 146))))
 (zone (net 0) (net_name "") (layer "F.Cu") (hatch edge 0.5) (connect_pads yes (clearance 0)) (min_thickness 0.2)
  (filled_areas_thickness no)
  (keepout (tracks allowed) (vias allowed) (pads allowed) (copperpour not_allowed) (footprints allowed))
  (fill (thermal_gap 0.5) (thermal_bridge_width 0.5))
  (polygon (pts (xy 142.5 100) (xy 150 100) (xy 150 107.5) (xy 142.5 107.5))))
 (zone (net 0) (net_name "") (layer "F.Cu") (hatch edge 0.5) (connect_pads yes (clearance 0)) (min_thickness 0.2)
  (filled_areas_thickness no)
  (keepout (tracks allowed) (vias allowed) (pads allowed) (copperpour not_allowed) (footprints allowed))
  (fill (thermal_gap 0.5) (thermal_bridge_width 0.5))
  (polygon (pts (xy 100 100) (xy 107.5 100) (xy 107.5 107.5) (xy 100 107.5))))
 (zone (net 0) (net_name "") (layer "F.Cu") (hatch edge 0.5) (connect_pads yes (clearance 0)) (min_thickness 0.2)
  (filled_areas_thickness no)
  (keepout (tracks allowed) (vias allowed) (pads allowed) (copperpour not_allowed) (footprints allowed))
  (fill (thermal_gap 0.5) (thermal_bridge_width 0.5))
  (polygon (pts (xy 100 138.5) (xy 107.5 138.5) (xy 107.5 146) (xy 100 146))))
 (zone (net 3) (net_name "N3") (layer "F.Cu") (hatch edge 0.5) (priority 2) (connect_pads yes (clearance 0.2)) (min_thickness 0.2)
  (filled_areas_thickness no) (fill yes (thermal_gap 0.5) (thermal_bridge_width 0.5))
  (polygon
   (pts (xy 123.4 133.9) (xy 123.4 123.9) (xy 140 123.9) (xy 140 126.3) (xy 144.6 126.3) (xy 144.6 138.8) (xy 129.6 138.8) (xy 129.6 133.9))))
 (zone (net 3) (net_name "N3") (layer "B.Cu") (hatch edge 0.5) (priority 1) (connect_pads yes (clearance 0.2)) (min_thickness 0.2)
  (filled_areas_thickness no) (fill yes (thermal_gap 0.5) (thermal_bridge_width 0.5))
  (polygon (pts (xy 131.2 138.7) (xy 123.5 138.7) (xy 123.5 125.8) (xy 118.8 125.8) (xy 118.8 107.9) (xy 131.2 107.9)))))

